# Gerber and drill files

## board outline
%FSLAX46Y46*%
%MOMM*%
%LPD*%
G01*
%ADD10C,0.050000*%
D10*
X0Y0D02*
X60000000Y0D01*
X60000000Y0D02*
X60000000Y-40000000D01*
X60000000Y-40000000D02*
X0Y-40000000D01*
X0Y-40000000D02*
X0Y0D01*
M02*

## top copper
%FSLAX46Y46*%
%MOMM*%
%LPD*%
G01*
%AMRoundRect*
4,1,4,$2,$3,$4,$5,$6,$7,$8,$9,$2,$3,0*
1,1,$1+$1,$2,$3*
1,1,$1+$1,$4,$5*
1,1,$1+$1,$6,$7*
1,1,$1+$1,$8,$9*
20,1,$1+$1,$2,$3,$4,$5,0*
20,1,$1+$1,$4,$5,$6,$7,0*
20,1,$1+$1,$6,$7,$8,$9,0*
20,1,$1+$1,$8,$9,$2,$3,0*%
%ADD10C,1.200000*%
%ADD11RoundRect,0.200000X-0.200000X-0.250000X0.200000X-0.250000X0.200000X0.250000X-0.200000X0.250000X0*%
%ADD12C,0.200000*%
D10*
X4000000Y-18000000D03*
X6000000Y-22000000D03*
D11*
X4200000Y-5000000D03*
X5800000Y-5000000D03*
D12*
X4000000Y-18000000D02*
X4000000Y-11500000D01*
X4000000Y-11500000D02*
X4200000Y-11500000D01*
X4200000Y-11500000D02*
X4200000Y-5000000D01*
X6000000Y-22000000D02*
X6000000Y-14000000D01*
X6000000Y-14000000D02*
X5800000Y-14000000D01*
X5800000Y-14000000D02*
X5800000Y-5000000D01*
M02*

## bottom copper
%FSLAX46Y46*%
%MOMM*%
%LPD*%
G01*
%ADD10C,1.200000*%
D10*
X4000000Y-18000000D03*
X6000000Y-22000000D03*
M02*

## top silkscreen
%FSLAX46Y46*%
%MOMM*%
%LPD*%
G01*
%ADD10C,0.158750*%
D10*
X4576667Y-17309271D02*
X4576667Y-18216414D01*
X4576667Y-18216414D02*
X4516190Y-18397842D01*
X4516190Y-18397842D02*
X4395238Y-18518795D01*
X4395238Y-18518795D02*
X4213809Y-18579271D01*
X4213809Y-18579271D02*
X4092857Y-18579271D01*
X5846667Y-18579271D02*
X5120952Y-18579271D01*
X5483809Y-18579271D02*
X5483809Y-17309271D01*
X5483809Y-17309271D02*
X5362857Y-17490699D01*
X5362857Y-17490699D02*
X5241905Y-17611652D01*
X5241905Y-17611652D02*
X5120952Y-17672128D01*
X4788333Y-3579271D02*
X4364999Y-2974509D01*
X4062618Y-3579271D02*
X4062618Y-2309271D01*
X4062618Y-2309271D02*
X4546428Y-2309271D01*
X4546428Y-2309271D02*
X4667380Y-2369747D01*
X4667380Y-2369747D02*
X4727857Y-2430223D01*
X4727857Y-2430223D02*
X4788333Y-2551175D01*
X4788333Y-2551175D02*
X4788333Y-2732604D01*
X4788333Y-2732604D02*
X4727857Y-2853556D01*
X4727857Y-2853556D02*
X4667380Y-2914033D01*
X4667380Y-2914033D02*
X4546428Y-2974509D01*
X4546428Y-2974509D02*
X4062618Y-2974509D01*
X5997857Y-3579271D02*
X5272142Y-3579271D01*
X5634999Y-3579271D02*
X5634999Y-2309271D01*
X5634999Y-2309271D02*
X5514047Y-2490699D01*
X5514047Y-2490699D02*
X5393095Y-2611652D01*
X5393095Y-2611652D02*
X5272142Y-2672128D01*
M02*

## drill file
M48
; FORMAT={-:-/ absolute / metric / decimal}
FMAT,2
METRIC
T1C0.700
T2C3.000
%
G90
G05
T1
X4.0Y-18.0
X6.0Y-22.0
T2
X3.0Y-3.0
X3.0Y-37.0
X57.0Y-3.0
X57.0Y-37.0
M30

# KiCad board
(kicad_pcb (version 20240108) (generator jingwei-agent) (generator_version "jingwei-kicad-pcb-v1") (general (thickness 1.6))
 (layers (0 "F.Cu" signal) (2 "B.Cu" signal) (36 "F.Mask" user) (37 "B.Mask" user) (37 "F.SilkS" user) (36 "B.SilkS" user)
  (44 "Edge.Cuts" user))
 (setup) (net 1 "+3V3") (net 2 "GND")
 (gr_line (start 0 0) (end 60 0) (stroke (width 0.05)) (layer "Edge.Cuts"))
 (gr_line (start 60 0) (end 60 40) (stroke (width 0.05)) (layer "Edge.Cuts"))
 (gr_line (start 60 40) (end 0 40) (stroke (width 0.05)) (layer "Edge.Cuts"))
 (gr_line (start 0 40) (end 0 0) (stroke (width 0.05)) (layer "Edge.Cuts"))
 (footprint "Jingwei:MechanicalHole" (layer "F.Cu") (at 3 3)
  (pad "" np_thru_hole circle (at 0 0) (size 3 3) (drill 3) (layers "*.Cu" "*.Mask")))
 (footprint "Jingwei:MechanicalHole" (layer "F.Cu") (at 57 3)
  (pad "" np_thru_hole circle (at 0 0) (size 3 3) (drill 3) (layers "*.Cu" "*.Mask")))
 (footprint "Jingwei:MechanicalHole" (layer "F.Cu") (at 3 37)
  (pad "" np_thru_hole circle (at 0 0) (size 3 3) (drill 3) (layers "*.Cu" "*.Mask")))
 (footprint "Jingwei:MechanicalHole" (layer "F.Cu") (at 57 37)
  (pad "" np_thru_hole circle (at 0 0) (size 3 3) (drill 3) (layers "*.Cu" "*.Mask")))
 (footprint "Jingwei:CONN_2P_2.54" (layer "F.Cu") (at 5 20) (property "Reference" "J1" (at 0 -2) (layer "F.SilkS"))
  (pad "1" thru_hole circle (at -1 -2) (size 1.2 1.2) (drill 0.7) (layers "*.Cu" "*.Mask") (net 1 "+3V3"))
  (pad "2" thru_hole circle (at 1 2) (size 1.2 1.2) (drill 0.7) (layers "*.Cu" "*.Mask") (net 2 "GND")))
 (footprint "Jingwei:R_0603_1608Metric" (layer "F.Cu") (at 5 5) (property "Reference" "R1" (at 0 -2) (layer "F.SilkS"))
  (pad "1" smd roundrect (at -0.8 0) (size 0.8 0.9) (layers "F.Cu" "F.Paste" "F.Mask") (roundrect_rratio 0.25) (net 1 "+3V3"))
  (pad "2" smd roundrect (at 0.8 0) (size 0.8 0.9) (layers "F.Cu" "F.Paste" "F.Mask") (roundrect_rratio 0.25) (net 2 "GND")))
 (segment (start 4 18) (end 4 11.5) (width 0.2) (layer "F.Cu") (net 1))
 (segment (start 4 11.5) (end 4.2 11.5) (width 0.2) (layer "F.Cu") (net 1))
 (segment (start 4.2 11.5) (end 4.2 5) (width 0.2) (layer "F.Cu") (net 1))
 (segment (start 6 22) (end 6 14) (width 0.2) (layer "F.Cu") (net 2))
 (segment (start 6 14) (end 5.8 14) (width 0.2) (layer "F.Cu") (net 2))
 (segment (start 5.8 14) (end 5.8 5) (width 0.2) (layer "F.Cu") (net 2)))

